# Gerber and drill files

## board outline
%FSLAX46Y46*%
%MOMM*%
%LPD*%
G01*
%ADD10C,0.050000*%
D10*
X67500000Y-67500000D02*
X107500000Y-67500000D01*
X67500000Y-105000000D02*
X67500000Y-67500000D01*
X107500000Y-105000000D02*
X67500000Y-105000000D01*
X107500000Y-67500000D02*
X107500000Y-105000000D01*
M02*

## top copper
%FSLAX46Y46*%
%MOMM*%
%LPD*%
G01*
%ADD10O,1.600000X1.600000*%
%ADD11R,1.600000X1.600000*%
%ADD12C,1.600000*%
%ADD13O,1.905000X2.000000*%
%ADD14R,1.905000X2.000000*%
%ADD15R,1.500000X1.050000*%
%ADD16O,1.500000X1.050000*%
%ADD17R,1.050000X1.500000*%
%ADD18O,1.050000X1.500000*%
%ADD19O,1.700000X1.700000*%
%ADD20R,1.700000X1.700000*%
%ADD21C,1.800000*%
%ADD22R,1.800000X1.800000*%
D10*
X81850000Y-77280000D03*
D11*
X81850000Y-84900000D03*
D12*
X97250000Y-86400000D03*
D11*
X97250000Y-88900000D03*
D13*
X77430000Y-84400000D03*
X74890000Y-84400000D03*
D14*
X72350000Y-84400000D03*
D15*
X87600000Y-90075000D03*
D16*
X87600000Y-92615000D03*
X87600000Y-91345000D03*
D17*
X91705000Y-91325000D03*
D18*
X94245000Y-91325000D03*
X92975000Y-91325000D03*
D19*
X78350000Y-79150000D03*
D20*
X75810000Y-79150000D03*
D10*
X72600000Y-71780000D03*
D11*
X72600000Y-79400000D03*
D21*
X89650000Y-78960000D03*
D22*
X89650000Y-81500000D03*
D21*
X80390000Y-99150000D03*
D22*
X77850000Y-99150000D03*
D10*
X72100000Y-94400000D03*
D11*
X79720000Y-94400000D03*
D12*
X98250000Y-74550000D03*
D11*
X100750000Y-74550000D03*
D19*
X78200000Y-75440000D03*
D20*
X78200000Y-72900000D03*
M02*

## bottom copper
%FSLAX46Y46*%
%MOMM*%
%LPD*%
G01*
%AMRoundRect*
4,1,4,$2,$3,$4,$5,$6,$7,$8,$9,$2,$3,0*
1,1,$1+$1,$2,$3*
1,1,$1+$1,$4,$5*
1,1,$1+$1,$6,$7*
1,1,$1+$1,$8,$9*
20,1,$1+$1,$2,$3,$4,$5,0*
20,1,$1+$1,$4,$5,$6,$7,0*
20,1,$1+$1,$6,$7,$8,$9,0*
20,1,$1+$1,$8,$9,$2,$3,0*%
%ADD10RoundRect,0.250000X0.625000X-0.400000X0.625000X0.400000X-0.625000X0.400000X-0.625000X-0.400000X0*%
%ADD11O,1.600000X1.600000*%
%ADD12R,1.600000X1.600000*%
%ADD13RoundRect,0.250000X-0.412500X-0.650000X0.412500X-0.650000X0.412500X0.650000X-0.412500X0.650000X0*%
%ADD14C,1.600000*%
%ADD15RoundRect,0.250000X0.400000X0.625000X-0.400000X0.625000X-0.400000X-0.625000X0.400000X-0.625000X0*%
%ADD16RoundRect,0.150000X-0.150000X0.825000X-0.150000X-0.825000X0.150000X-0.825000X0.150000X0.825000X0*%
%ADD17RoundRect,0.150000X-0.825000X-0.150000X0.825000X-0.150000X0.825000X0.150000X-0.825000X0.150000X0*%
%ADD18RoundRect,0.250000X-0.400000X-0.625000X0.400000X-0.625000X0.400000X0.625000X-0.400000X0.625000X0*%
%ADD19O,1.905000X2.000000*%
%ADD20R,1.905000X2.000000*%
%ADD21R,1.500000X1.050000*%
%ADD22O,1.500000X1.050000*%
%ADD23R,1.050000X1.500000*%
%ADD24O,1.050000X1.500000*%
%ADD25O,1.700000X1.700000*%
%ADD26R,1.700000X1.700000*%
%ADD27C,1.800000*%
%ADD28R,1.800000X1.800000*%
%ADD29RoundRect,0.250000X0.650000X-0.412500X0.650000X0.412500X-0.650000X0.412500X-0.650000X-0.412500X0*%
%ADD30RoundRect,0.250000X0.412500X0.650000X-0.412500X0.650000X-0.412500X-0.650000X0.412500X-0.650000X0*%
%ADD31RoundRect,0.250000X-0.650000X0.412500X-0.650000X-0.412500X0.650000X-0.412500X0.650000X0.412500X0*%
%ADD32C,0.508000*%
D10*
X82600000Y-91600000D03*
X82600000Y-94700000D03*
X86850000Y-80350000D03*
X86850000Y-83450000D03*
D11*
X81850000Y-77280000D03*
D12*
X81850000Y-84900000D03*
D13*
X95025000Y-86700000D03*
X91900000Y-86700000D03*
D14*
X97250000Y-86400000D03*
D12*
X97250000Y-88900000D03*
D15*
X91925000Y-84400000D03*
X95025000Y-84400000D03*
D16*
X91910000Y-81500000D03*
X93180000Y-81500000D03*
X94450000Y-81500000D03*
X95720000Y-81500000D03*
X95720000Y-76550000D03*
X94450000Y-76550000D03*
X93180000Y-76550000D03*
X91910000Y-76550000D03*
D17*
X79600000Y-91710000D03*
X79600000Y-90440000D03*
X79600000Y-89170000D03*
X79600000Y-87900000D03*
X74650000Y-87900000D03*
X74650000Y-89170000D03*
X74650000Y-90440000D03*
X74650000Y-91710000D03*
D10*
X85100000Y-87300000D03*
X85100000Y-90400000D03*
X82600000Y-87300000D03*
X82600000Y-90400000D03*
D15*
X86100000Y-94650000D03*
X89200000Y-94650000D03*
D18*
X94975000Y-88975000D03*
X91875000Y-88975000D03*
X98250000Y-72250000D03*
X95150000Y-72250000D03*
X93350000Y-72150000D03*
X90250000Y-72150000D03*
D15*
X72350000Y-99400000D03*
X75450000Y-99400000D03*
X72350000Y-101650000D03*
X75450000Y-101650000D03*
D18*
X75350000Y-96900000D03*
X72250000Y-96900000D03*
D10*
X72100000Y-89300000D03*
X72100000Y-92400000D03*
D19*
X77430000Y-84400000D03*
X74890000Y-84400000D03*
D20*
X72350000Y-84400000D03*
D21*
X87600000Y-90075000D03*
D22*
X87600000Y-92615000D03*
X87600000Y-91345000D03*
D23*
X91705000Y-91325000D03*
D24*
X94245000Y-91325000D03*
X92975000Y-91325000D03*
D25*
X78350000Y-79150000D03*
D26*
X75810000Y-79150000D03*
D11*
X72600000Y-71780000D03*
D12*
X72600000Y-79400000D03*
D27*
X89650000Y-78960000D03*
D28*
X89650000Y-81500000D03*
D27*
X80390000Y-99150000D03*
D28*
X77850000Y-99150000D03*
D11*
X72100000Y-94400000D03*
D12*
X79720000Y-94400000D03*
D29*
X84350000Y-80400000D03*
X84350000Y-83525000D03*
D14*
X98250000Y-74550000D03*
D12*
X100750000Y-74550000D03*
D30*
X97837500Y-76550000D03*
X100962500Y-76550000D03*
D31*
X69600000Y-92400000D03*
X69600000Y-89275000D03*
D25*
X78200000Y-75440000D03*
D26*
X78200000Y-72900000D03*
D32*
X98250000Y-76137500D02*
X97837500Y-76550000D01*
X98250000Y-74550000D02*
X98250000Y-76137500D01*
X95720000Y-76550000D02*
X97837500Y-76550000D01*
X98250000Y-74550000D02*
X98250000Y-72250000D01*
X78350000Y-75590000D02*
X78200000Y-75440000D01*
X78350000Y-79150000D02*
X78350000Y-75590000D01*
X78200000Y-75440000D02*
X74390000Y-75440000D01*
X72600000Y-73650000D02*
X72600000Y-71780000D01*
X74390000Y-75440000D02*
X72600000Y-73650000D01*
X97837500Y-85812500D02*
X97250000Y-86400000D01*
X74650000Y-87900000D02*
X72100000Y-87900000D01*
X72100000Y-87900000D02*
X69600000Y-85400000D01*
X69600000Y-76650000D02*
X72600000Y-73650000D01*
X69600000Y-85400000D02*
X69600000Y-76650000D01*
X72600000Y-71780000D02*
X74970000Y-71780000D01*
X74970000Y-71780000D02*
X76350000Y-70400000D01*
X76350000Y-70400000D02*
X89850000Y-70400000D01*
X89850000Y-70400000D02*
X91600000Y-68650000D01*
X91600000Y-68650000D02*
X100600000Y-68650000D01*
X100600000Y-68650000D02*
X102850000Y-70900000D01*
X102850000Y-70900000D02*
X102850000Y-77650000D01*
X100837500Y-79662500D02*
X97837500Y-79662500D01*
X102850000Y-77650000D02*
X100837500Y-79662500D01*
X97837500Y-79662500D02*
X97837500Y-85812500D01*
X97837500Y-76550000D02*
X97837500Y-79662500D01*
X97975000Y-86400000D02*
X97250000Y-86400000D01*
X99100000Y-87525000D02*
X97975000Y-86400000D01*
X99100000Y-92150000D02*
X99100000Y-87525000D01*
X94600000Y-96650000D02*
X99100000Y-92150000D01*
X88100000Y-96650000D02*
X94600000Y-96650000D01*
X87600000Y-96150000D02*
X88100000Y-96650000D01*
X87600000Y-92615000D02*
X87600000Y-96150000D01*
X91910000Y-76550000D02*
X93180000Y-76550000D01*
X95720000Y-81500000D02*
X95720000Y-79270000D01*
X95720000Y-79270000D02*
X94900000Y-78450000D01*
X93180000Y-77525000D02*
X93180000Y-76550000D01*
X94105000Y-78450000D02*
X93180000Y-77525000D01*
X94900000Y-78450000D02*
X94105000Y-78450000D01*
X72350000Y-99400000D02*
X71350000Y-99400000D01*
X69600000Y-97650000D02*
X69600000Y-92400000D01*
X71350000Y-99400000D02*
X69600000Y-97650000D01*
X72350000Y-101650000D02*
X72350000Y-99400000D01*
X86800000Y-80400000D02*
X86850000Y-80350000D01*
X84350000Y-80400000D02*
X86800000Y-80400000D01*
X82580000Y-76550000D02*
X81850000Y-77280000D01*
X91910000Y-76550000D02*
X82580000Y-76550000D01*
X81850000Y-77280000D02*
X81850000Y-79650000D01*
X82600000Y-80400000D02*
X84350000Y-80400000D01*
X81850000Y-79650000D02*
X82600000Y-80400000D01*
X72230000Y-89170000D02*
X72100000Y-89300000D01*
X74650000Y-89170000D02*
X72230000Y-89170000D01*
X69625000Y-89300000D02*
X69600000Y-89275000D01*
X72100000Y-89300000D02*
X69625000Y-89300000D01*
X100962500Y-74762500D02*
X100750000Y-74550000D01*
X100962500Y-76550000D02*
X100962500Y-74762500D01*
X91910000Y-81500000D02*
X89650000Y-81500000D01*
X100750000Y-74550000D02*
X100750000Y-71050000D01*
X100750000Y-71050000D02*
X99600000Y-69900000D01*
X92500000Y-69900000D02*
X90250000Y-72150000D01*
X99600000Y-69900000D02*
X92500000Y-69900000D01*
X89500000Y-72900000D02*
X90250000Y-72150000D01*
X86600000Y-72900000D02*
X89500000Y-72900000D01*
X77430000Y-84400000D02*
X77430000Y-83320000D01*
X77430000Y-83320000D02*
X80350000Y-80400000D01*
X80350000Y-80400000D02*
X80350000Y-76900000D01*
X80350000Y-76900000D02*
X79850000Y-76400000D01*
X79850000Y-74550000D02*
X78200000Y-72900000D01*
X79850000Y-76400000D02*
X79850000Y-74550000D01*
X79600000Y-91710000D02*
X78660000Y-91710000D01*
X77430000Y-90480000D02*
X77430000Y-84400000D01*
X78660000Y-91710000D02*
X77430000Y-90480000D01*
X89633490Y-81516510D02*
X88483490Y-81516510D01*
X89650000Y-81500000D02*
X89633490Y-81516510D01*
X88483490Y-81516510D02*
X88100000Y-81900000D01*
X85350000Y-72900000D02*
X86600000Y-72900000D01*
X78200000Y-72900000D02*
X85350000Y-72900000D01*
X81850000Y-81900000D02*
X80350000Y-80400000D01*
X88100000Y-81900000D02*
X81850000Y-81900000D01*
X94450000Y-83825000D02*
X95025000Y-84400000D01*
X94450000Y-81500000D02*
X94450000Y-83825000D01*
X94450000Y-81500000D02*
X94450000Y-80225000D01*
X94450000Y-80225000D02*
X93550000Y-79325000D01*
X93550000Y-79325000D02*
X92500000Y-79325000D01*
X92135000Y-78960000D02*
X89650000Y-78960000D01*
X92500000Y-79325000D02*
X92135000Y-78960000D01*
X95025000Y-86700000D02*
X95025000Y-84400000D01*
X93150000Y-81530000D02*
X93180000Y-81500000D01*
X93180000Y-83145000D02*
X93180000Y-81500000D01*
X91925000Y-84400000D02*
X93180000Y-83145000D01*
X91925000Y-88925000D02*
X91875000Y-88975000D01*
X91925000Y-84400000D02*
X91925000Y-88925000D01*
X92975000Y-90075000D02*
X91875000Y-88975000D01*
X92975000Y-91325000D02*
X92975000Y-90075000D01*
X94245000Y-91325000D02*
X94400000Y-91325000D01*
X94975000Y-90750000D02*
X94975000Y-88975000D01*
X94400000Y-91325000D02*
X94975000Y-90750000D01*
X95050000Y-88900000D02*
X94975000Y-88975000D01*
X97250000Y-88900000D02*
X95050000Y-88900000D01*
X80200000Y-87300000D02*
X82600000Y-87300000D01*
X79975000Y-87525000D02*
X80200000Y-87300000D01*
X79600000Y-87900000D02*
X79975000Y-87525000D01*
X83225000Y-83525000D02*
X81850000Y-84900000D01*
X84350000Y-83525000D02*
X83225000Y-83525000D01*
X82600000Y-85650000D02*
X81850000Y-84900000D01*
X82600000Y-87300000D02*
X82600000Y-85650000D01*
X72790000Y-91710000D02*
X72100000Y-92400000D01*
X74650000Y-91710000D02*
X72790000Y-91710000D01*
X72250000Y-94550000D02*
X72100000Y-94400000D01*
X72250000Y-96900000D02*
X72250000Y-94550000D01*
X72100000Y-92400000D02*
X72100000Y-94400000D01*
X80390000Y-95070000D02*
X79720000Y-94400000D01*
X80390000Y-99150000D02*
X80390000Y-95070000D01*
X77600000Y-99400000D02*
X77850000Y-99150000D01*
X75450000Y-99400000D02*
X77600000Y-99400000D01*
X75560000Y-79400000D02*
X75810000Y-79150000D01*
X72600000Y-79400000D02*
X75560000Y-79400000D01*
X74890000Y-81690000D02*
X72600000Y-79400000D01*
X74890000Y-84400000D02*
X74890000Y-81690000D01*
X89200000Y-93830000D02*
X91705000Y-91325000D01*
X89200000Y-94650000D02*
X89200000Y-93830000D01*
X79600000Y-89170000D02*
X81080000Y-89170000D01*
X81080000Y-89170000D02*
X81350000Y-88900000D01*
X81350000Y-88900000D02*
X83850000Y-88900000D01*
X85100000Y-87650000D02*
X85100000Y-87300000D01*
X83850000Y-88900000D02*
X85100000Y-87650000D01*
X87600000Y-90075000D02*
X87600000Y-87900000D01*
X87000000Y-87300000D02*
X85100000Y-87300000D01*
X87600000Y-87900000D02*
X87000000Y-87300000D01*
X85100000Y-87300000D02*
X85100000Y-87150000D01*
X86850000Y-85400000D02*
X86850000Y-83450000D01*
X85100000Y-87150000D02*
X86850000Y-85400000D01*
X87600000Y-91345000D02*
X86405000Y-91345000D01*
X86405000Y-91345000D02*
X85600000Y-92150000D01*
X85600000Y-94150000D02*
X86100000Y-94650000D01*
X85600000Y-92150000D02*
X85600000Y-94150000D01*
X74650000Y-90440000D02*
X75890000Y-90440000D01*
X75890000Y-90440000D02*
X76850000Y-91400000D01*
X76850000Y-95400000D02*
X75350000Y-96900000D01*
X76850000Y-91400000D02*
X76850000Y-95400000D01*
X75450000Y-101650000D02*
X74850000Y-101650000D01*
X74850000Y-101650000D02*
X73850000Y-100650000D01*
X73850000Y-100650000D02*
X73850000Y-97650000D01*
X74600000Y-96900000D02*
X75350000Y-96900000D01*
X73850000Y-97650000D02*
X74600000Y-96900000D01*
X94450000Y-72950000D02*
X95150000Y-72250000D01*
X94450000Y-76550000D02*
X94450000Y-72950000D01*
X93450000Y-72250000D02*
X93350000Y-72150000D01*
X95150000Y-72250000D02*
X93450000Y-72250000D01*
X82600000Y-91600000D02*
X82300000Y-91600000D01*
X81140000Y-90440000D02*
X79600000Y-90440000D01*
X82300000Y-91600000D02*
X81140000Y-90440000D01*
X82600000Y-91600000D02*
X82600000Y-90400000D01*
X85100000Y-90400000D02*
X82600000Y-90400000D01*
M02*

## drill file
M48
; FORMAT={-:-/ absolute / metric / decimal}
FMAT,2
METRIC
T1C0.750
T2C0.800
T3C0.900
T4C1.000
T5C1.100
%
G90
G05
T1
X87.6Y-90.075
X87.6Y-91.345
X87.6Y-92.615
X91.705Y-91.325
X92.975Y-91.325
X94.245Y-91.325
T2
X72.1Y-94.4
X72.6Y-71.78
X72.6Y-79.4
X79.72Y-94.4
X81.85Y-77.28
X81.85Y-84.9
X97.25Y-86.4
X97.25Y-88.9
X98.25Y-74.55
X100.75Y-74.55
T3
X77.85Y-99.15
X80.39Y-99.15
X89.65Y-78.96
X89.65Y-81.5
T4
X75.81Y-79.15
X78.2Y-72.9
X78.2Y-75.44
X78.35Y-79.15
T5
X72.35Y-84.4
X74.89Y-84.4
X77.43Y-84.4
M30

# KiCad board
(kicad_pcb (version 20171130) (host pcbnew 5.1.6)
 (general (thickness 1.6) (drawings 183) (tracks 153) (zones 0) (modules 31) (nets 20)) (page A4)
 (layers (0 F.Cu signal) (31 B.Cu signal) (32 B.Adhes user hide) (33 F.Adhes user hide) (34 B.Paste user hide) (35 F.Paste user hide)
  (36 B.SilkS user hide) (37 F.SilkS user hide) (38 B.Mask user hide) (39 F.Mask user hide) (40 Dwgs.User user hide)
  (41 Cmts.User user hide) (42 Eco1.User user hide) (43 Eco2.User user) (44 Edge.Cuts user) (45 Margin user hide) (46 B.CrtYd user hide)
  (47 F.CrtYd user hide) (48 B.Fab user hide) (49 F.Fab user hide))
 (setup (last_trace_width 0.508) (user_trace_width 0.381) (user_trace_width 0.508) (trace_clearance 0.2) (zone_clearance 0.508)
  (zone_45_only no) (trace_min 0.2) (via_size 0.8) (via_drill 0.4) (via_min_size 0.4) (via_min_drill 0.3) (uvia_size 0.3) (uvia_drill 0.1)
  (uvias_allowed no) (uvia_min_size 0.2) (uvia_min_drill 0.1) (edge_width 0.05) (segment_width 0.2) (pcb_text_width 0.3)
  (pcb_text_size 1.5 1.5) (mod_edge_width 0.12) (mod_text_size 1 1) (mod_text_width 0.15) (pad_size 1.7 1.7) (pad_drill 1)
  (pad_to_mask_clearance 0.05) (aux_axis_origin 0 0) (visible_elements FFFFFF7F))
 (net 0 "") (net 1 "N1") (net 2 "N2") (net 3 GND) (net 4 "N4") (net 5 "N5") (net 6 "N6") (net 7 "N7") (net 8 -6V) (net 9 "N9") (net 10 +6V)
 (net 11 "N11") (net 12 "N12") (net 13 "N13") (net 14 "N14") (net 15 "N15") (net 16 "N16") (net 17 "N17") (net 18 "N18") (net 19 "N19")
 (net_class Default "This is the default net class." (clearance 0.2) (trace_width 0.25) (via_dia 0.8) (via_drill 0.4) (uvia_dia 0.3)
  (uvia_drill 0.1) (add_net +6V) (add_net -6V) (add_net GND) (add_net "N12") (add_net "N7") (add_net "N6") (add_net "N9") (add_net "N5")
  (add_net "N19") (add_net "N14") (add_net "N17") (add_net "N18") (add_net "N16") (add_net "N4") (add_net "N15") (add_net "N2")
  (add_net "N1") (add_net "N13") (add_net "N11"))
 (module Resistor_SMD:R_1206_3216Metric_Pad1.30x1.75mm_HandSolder (layer B.Cu) (at 82.6 93.15 90)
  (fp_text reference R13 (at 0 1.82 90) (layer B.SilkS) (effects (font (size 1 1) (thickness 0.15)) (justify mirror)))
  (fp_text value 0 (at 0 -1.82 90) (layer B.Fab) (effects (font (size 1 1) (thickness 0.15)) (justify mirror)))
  (pad 2 smd roundrect (at 1.55 0 90) (size 1.3 1.75) (layers B.Cu B.Paste B.Mask) (roundrect_rratio 0.192308) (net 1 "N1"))
  (pad 1 smd roundrect (at -1.55 0 90) (size 1.3 1.75) (layers B.Cu B.Paste B.Mask) (roundrect_rratio 0.192308) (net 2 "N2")))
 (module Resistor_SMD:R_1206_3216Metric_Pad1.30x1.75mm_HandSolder (layer B.Cu) (at 86.85 81.9 90)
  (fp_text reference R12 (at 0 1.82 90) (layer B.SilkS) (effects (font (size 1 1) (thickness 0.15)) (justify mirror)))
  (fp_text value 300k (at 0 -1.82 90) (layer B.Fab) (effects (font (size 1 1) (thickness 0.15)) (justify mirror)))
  (pad 2 smd roundrect (at 1.55 0 90) (size 1.3 1.75) (layers B.Cu B.Paste B.Mask) (roundrect_rratio 0.192308) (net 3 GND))
  (pad 1 smd roundrect (at -1.55 0 90) (size 1.3 1.75) (layers B.Cu B.Paste B.Mask) (roundrect_rratio 0.192308) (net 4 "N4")))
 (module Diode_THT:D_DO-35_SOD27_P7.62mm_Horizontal (layer F.Cu) (at 81.85 84.9 90)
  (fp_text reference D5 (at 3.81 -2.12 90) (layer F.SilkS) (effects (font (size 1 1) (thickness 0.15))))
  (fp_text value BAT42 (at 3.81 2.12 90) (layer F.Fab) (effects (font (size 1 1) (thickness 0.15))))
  (pad 2 thru_hole oval (at 7.62 0 90) (size 1.6 1.6) (drill 0.8) (layers *.Cu *.Mask) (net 3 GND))
  (pad 1 thru_hole rect (at 0 0 90) (size 1.6 1.6) (drill 0.8) (layers *.Cu *.Mask) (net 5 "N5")))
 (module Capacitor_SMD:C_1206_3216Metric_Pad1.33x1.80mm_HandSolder (layer B.Cu) (at 93.4625 86.7)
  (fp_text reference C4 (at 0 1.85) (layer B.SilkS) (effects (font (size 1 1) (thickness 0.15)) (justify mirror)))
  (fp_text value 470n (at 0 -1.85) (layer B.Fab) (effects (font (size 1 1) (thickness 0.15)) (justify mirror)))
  (pad 2 smd roundrect (at 1.5625 0) (size 1.325 1.8) (layers B.Cu B.Paste B.Mask) (roundrect_rratio 0.188679) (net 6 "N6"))
  (pad 1 smd roundrect (at -1.5625 0) (size 1.325 1.8) (layers B.Cu B.Paste B.Mask) (roundrect_rratio 0.188679) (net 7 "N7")))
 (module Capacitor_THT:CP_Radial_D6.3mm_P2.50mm (layer F.Cu) (at 97.25 88.9 90)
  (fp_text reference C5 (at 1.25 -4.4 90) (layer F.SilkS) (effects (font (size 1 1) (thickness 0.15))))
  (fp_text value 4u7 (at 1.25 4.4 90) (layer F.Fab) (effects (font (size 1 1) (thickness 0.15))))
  (pad 2 thru_hole circle (at 2.5 0 90) (size 1.6 1.6) (drill 0.8) (layers *.Cu *.Mask) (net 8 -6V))
  (pad 1 thru_hole rect (at 0 0 90) (size 1.6 1.6) (drill 0.8) (layers *.Cu *.Mask) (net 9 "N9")))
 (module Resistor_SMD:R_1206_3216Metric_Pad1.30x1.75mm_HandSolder (layer B.Cu) (at 93.475 84.4 180)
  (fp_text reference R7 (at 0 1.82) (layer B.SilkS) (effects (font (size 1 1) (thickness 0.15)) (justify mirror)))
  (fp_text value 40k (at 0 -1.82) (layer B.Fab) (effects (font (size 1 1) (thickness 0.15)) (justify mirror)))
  (pad 2 smd roundrect (at 1.55 0 180) (size 1.3 1.75) (layers B.Cu B.Paste B.Mask) (roundrect_rratio 0.192308) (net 7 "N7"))
  (pad 1 smd roundrect (at -1.55 0 180) (size 1.3 1.75) (layers B.Cu B.Paste B.Mask) (roundrect_rratio 0.192308) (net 6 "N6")))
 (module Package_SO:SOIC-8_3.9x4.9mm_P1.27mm (layer B.Cu) (at 93.815 79.025 270)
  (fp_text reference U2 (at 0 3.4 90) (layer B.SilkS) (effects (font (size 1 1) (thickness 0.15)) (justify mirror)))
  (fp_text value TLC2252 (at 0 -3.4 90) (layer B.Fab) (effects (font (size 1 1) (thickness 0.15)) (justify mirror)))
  (pad 8 smd roundrect (at 2.475 1.905 270) (size 1.95 0.6) (layers B.Cu B.Paste B.Mask) (roundrect_rratio 0.25) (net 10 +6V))
  (pad 7 smd roundrect (at 2.475 0.635 270) (size 1.95 0.6) (layers B.Cu B.Paste B.Mask) (roundrect_rratio 0.25) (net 7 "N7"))
  (pad 6 smd roundrect (at 2.475 -0.635 270) (size 1.95 0.6) (layers B.Cu B.Paste B.Mask) (roundrect_rratio 0.25) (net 6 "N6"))
  (pad 5 smd roundrect (at 2.475 -1.905 270) (size 1.95 0.6) (layers B.Cu B.Paste B.Mask) (roundrect_rratio 0.25) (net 3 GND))
  (pad 4 smd roundrect (at -2.475 -1.905 270) (size 1.95 0.6) (layers B.Cu B.Paste B.Mask) (roundrect_rratio 0.25) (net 8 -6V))
  (pad 3 smd roundrect (at -2.475 -0.635 270) (size 1.95 0.6) (layers B.Cu B.Paste B.Mask) (roundrect_rratio 0.25) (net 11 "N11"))
  (pad 2 smd roundrect (at -2.475 0.635 270) (size 1.95 0.6) (layers B.Cu B.Paste B.Mask) (roundrect_rratio 0.25) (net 3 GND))
  (pad 1 smd roundrect (at -2.475 1.905 270) (size 1.95 0.6) (layers B.Cu B.Paste B.Mask) (roundrect_rratio 0.25) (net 3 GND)))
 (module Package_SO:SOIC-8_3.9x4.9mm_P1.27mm (layer B.Cu) (at 77.125 89.805)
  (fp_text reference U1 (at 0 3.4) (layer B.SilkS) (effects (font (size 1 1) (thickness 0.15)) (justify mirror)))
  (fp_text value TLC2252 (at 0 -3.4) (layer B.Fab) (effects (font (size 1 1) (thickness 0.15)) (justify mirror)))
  (pad 8 smd roundrect (at 2.475 1.905) (size 1.95 0.6) (layers B.Cu B.Paste B.Mask) (roundrect_rratio 0.25) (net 10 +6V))
  (pad 7 smd roundrect (at 2.475 0.635) (size 1.95 0.6) (layers B.Cu B.Paste B.Mask) (roundrect_rratio 0.25) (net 1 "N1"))
  (pad 6 smd roundrect (at 2.475 -0.635) (size 1.95 0.6) (layers B.Cu B.Paste B.Mask) (roundrect_rratio 0.25) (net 4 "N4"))
  (pad 5 smd roundrect (at 2.475 -1.905) (size 1.95 0.6) (layers B.Cu B.Paste B.Mask) (roundrect_rratio 0.25) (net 5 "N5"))
  (pad 4 smd roundrect (at -2.475 -1.905) (size 1.95 0.6) (layers B.Cu B.Paste B.Mask) (roundrect_rratio 0.25) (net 8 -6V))
  (pad 3 smd roundrect (at -2.475 -0.635) (size 1.95 0.6) (layers B.Cu B.Paste B.Mask) (roundrect_rratio 0.25) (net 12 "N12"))
  (pad 2 smd roundrect (at -2.475 0.635) (size 1.95 0.6) (layers B.Cu B.Paste B.Mask) (roundrect_rratio 0.25) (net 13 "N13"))
  (pad 1 smd roundrect (at -2.475 1.905) (size 1.95 0.6) (layers B.Cu B.Paste B.Mask) (roundrect_rratio 0.25) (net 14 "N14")))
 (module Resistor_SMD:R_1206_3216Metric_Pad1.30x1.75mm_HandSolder (layer B.Cu) (at 85.1 88.85 90)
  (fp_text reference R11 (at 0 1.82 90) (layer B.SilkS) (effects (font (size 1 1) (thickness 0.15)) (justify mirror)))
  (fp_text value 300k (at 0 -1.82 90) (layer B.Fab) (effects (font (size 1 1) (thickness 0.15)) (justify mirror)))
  (pad 2 smd roundrect (at 1.55 0 90) (size 1.3 1.75) (layers B.Cu B.Paste B.Mask) (roundrect_rratio 0.192308) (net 4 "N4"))
  (pad 1 smd roundrect (at -1.55 0 90) (size 1.3 1.75) (layers B.Cu B.Paste B.Mask) (roundrect_rratio 0.192308) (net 1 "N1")))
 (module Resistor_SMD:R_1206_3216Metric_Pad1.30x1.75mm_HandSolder (layer B.Cu) (at 82.6 88.85 90)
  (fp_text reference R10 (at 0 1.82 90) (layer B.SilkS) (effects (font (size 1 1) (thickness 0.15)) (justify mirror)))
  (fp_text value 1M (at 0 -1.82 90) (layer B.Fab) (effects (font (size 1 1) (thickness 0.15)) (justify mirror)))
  (pad 2 smd roundrect (at 1.55 0 90) (size 1.3 1.75) (layers B.Cu B.Paste B.Mask) (roundrect_rratio 0.192308) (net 5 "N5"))
  (pad 1 smd roundrect (at -1.55 0 90) (size 1.3 1.75) (layers B.Cu B.Paste B.Mask) (roundrect_rratio 0.192308) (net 1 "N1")))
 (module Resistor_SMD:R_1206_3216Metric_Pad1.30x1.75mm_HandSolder (layer B.Cu) (at 87.65 94.65 180)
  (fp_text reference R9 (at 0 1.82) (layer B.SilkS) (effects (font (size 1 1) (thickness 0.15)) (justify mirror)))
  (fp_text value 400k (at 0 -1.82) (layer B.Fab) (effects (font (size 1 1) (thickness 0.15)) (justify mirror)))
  (pad 2 smd roundrect (at 1.55 0 180) (size 1.3 1.75) (layers B.Cu B.Paste B.Mask) (roundrect_rratio 0.192308) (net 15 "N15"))
  (pad 1 smd roundrect (at -1.55 0 180) (size 1.3 1.75) (layers B.Cu B.Paste B.Mask) (roundrect_rratio 0.192308) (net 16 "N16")))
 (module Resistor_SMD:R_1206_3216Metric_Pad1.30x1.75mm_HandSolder (layer B.Cu) (at 93.425 88.975)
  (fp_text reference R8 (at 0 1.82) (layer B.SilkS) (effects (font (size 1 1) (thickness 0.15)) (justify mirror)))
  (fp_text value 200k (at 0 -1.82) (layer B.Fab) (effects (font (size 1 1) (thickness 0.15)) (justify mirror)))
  (pad 2 smd roundrect (at 1.55 0) (size 1.3 1.75) (layers B.Cu B.Paste B.Mask) (roundrect_rratio 0.192308) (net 9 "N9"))
  (pad 1 smd roundrect (at -1.55 0) (size 1.3 1.75) (layers B.Cu B.Paste B.Mask) (roundrect_rratio 0.192308) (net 7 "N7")))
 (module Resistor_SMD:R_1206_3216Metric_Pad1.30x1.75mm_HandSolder (layer B.Cu) (at 96.7 72.25)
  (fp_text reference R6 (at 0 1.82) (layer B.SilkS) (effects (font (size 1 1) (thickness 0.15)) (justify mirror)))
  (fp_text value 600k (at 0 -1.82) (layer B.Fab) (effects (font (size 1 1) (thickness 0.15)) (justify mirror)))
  (pad 2 smd roundrect (at 1.55 0) (size 1.3 1.75) (layers B.Cu B.Paste B.Mask) (roundrect_rratio 0.192308) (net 8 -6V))
  (pad 1 smd roundrect (at -1.55 0) (size 1.3 1.75) (layers B.Cu B.Paste B.Mask) (roundrect_rratio 0.192308) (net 11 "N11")))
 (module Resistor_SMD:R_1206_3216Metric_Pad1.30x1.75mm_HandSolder (layer B.Cu) (at 91.8 72.15)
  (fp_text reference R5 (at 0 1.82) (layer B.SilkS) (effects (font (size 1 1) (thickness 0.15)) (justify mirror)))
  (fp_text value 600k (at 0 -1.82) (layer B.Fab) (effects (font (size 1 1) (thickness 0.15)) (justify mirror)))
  (pad 2 smd roundrect (at 1.55 0) (size 1.3 1.75) (layers B.Cu B.Paste B.Mask) (roundrect_rratio 0.192308) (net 11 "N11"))
  (pad 1 smd roundrect (at -1.55 0) (size 1.3 1.75) (layers B.Cu B.Paste B.Mask) (roundrect_rratio 0.192308) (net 10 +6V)))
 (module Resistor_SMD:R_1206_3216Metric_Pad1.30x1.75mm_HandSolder (layer B.Cu) (at 73.9 99.4 180)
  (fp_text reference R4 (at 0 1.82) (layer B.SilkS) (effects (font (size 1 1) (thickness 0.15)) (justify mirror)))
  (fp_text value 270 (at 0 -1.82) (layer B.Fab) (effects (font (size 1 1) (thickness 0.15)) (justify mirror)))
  (pad 2 smd roundrect (at 1.55 0 180) (size 1.3 1.75) (layers B.Cu B.Paste B.Mask) (roundrect_rratio 0.192308) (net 3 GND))
  (pad 1 smd roundrect (at -1.55 0 180) (size 1.3 1.75) (layers B.Cu B.Paste B.Mask) (roundrect_rratio 0.192308) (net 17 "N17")))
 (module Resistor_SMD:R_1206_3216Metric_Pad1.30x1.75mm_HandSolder (layer B.Cu) (at 73.9 101.65 180)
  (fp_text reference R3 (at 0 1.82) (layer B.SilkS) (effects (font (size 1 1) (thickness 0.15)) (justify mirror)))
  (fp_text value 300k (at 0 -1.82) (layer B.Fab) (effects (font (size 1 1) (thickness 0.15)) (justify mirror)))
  (pad 2 smd roundrect (at 1.55 0 180) (size 1.3 1.75) (layers B.Cu B.Paste B.Mask) (roundrect_rratio 0.192308) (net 3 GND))
  (pad 1 smd roundrect (at -1.55 0 180) (size 1.3 1.75) (layers B.Cu B.Paste B.Mask) (roundrect_rratio 0.192308) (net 13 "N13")))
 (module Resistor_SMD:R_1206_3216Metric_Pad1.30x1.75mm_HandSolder (layer B.Cu) (at 73.8 96.9)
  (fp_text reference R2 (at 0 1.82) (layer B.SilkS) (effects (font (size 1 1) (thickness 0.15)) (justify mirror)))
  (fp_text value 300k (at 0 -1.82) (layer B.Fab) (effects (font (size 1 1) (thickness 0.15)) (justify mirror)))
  (pad 2 smd roundrect (at 1.55 0) (size 1.3 1.75) (layers B.Cu B.Paste B.Mask) (roundrect_rratio 0.192308) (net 13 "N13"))
  (pad 1 smd roundrect (at -1.55 0) (size 1.3 1.75) (layers B.Cu B.Paste B.Mask) (roundrect_rratio 0.192308) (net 14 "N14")))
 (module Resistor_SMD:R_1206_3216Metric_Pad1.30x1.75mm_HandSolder (layer B.Cu) (at 72.1 90.85 90)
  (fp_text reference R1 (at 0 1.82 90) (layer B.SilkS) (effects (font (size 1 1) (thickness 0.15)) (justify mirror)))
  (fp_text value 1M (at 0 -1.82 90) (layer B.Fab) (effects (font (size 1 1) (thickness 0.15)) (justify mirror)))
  (pad 2 smd roundrect (at 1.55 0 90) (size 1.3 1.75) (layers B.Cu B.Paste B.Mask) (roundrect_rratio 0.192308) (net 12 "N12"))
  (pad 1 smd roundrect (at -1.55 0 90) (size 1.3 1.75) (layers B.Cu B.Paste B.Mask) (roundrect_rratio 0.192308) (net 14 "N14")))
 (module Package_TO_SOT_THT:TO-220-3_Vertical (layer F.Cu) (at 72.35 84.4)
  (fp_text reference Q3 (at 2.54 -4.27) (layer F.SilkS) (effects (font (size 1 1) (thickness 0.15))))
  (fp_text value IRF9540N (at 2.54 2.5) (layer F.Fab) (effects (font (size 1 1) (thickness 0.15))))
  (pad 3 thru_hole oval (at 5.08 0) (size 1.905 2) (drill 1.1) (layers *.Cu *.Mask) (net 10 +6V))
  (pad 2 thru_hole oval (at 2.54 0) (size 1.905 2) (drill 1.1) (layers *.Cu *.Mask) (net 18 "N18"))
  (pad 1 thru_hole rect (at 0 0) (size 1.905 2) (drill 1.1) (layers *.Cu *.Mask) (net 2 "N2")))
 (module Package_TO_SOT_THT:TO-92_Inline (layer F.Cu) (at 87.6 90.075 270)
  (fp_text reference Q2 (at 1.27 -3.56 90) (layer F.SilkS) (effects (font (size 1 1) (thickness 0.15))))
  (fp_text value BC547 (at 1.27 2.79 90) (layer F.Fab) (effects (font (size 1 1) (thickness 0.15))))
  (pad 1 thru_hole rect (at 0 0 270) (size 1.05 1.5) (drill 0.75) (layers *.Cu *.Mask) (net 4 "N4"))
  (pad 3 thru_hole oval (at 2.54 0 270) (size 1.05 1.5) (drill 0.75) (layers *.Cu *.Mask) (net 8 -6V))
  (pad 2 thru_hole oval (at 1.27 0 270) (size 1.05 1.5) (drill 0.75) (layers *.Cu *.Mask) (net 15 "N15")))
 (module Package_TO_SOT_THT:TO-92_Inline (layer F.Cu) (at 91.705 91.325)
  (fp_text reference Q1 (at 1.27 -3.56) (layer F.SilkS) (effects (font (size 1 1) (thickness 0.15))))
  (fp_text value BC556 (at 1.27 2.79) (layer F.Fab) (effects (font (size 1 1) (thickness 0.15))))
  (pad 1 thru_hole rect (at 0 0) (size 1.05 1.5) (drill 0.75) (layers *.Cu *.Mask) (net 16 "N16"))
  (pad 3 thru_hole oval (at 2.54 0) (size 1.05 1.5) (drill 0.75) (layers *.Cu *.Mask) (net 9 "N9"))
  (pad 2 thru_hole oval (at 1.27 0) (size 1.05 1.5) (drill 0.75) (layers *.Cu *.Mask) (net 7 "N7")))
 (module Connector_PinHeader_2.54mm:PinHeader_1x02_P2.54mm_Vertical (layer F.Cu) (at 75.81 79.15 90)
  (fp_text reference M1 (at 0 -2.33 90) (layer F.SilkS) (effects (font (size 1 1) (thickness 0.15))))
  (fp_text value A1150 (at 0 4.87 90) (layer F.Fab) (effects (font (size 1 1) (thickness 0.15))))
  (pad 2 thru_hole oval (at 0 2.54 90) (size 1.7 1.7) (drill 1) (layers *.Cu *.Mask) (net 8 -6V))
  (pad 1 thru_hole rect (at 0 0 90) (size 1.7 1.7) (drill 1) (layers *.Cu *.Mask) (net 18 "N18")))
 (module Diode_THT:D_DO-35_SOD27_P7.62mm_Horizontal (layer F.Cu) (at 72.6 79.4 90)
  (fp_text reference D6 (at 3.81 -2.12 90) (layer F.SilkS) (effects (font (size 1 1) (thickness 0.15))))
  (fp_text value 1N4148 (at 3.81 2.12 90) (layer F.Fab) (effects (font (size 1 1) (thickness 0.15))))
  (pad 2 thru_hole oval (at 7.62 0 90) (size 1.6 1.6) (drill 0.8) (layers *.Cu *.Mask) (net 8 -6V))
  (pad 1 thru_hole rect (at 0 0 90) (size 1.6 1.6) (drill 0.8) (layers *.Cu *.Mask) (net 18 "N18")))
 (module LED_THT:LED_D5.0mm (layer F.Cu) (at 89.65 81.5 90)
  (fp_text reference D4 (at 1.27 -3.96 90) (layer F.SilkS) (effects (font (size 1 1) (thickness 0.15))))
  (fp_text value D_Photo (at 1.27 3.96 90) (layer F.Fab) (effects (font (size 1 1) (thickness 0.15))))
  (pad 2 thru_hole circle (at 2.54 0 90) (size 1.8 1.8) (drill 0.9) (layers *.Cu *.Mask) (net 6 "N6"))
  (pad 1 thru_hole rect (at 0 0 90) (size 1.8 1.8) (drill 0.9) (layers *.Cu *.Mask) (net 10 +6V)))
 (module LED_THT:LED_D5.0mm (layer F.Cu) (at 77.85 99.15)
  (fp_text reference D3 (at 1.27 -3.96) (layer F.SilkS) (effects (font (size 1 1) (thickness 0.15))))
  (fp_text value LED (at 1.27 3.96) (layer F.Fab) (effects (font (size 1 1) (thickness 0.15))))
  (pad 2 thru_hole circle (at 2.54 0) (size 1.8 1.8) (drill 0.9) (layers *.Cu *.Mask) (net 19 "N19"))
  (pad 1 thru_hole rect (at 0 0) (size 1.8 1.8) (drill 0.9) (layers *.Cu *.Mask) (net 17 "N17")))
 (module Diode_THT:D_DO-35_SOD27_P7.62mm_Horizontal (layer F.Cu) (at 79.72 94.4 180)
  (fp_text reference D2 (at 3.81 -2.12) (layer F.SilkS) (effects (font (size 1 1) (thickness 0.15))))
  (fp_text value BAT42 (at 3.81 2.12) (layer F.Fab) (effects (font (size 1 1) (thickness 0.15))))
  (pad 2 thru_hole oval (at 7.62 0 180) (size 1.6 1.6) (drill 0.8) (layers *.Cu *.Mask) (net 14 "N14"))
  (pad 1 thru_hole rect (at 0 0 180) (size 1.6 1.6) (drill 0.8) (layers *.Cu *.Mask) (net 19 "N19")))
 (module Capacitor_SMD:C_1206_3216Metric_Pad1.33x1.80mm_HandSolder (layer B.Cu) (at 84.35 81.9625 90)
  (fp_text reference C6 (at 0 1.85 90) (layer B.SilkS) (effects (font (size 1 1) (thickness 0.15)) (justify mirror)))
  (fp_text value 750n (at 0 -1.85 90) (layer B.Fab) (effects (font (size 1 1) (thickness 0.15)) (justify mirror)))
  (pad 2 smd roundrect (at 1.5625 0 90) (size 1.325 1.8) (layers B.Cu B.Paste B.Mask) (roundrect_rratio 0.188679) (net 3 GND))
  (pad 1 smd roundrect (at -1.5625 0 90) (size 1.325 1.8) (layers B.Cu B.Paste B.Mask) (roundrect_rratio 0.188679) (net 5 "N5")))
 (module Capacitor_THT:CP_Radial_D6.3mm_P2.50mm (layer F.Cu) (at 100.75 74.55 180)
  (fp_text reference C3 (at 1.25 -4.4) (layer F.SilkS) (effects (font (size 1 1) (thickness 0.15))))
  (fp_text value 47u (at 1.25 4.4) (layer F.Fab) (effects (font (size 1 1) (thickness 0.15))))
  (pad 2 thru_hole circle (at 2.5 0 180) (size 1.6 1.6) (drill 0.8) (layers *.Cu *.Mask) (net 8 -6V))
  (pad 1 thru_hole rect (at 0 0 180) (size 1.6 1.6) (drill 0.8) (layers *.Cu *.Mask) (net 10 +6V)))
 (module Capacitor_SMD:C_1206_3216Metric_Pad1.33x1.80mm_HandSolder (layer B.Cu) (at 99.4 76.55 180)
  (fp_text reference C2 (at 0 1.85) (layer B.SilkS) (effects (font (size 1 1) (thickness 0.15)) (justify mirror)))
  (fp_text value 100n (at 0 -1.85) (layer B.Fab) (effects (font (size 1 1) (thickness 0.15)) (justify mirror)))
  (pad 2 smd roundrect (at 1.5625 0 180) (size 1.325 1.8) (layers B.Cu B.Paste B.Mask) (roundrect_rratio 0.188679) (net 8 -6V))
  (pad 1 smd roundrect (at -1.5625 0 180) (size 1.325 1.8) (layers B.Cu B.Paste B.Mask) (roundrect_rratio 0.188679) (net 10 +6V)))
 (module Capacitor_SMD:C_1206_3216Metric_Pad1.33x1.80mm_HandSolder (layer B.Cu) (at 69.6 90.8375 270)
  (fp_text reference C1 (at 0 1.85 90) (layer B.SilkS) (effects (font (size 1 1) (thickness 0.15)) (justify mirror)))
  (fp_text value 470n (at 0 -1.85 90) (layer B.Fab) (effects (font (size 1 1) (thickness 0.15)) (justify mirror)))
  (pad 2 smd roundrect (at 1.5625 0 270) (size 1.325 1.8) (layers B.Cu B.Paste B.Mask) (roundrect_rratio 0.188679) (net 3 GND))
  (pad 1 smd roundrect (at -1.5625 0 270) (size 1.325 1.8) (layers B.Cu B.Paste B.Mask) (roundrect_rratio 0.188679) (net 12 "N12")))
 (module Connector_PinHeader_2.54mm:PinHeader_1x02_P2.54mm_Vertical (layer F.Cu) (at 78.2 72.9)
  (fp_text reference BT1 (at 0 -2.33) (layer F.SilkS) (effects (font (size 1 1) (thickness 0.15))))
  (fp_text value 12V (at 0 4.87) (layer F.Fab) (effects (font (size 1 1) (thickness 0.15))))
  (pad 2 thru_hole oval (at 0 2.54) (size 1.7 1.7) (drill 1) (layers *.Cu *.Mask) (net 8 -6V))
  (pad 1 thru_hole rect (at 0 0) (size 1.7 1.7) (drill 1) (layers *.Cu *.Mask) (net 10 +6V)))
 (gr_line (start 67.5 67.5) (end 107.5 67.5) (layer Edge.Cuts) (width 0.05))
 (gr_line (start 67.5 105) (end 67.5 67.5) (layer Edge.Cuts) (width 0.05))
 (gr_line (start 107.5 105) (end 67.5 105) (layer Edge.Cuts) (width 0.05))
 (gr_line (start 107.5 67.5) (end 107.5 105) (layer Edge.Cuts) (width 0.05))
 (segment (start 98.25 76.1375) (end 97.8375 76.55) (width 0.508) (layer B.Cu) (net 8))
 (segment (start 98.25 74.55) (end 98.25 76.1375) (width 0.508) (layer B.Cu) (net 8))
 (segment (start 95.72 76.55) (end 97.8375 76.55) (width 0.508) (layer B.Cu) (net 8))
 (segment (start 98.25 74.55) (end 98.25 72.25) (width 0.508) (layer B.Cu) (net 8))
 (segment (start 78.35 75.59) (end 78.2 75.44) (width 0.508) (layer B.Cu) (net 8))
 (segment (start 78.35 79.15) (end 78.35 75.59) (width 0.508) (layer B.Cu) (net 8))
 (segment (start 78.2 75.44) (end 74.39 75.44) (width 0.508) (layer B.Cu) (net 8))
 (segment (start 72.6 73.65) (end 72.6 71.78) (width 0.508) (layer B.Cu) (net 8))
 (segment (start 74.39 75.44) (end 72.6 73.65) (width 0.508) (layer B.Cu) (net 8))
 (segment (start 97.8375 85.8125) (end 97.25 86.4) (width 0.508) (layer B.Cu) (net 8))
 (segment (start 74.65 87.9) (end 72.1 87.9) (width 0.508) (layer B.Cu) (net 8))
 (segment (start 72.1 87.9) (end 69.6 85.4) (width 0.508) (layer B.Cu) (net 8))
 (segment (start 69.6 76.65) (end 72.6 73.65) (width 0.508) (layer B.Cu) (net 8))
 (segment (start 69.6 85.4) (end 69.6 76.65) (width 0.508) (layer B.Cu) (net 8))
 (segment (start 72.6 71.78) (end 74.97 71.78) (width 0.508) (layer B.Cu) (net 8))
 (segment (start 74.97 71.78) (end 76.35 70.4) (width 0.508) (layer B.Cu) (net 8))
 (segment (start 76.35 70.4) (end 89.85 70.4) (width 0.508) (layer B.Cu) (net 8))
 (segment (start 89.85 70.4) (end 91.6 68.65) (width 0.508) (layer B.Cu) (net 8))
 (segment (start 91.6 68.65) (end 100.6 68.65) (width 0.508) (layer B.Cu) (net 8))
 (segment (start 100.6 68.65) (end 102.85 70.9) (width 0.508) (layer B.Cu) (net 8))
 (segment (start 102.85 70.9) (end 102.85 77.65) (width 0.508) (layer B.Cu) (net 8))
 (segment (start 100.8375 79.6625) (end 97.8375 79.6625) (width 0.508) (layer B.Cu) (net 8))
 (segment (start 102.85 77.65) (end 100.8375 79.6625) (width 0.508) (layer B.Cu) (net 8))
 (segment (start 97.8375 79.6625) (end 97.8375 85.8125) (width 0.508) (layer B.Cu) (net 8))
 (segment (start 97.8375 76.55) (end 97.8375 79.6625) (width 0.508) (layer B.Cu) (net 8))
 (segment (start 97.975 86.4) (end 97.25 86.4) (width 0.508) (layer B.Cu) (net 8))
 (segment (start 99.1 87.525) (end 97.975 86.4) (width 0.508) (layer B.Cu) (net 8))
 (segment (start 99.1 92.15) (end 99.1 87.525) (width 0.508) (layer B.Cu) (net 8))
 (segment (start 94.6 96.65) (end 99.1 92.15) (width 0.508) (layer B.Cu) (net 8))
 (segment (start 88.1 96.65) (end 94.6 96.65) (width 0.508) (layer B.Cu) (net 8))
 (segment (start 87.6 96.15) (end 88.1 96.65) (width 0.508) (layer B.Cu) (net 8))
 (segment (start 87.6 92.615) (end 87.6 96.15) (width 0.508) (layer B.Cu) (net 8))
 (segment (start 91.91 76.55) (end 93.18 76.55) (width 0.508) (layer B.Cu) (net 3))
 (segment (start 95.72 81.5) (end 95.72 79.27) (width 0.508) (layer B.Cu) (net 3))
 (segment (start 95.72 79.27) (end 94.9 78.45) (width 0.508) (layer B.Cu) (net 3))
 (segment (start 93.18 77.525) (end 93.18 76.55) (width 0.508) (layer B.Cu) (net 3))
 (segment (start 94.105 78.45) (end 93.18 77.525) (width 0.508) (layer B.Cu) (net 3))
 (segment (start 94.9 78.45) (end 94.105 78.45) (width 0.508) (layer B.Cu) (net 3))
 (segment (start 72.35 99.4) (end 71.35 99.4) (width 0.508) (layer B.Cu) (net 3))
 (segment (start 69.6 97.65) (end 69.6 92.4) (width 0.508) (layer B.Cu) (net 3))
 (segment (start 71.35 99.4) (end 69.6 97.65) (width 0.508) (layer B.Cu) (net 3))
 (segment (start 72.35 101.65) (end 72.35 99.4) (width 0.508) (layer B.Cu) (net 3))
 (segment (start 86.8 80.4) (end 86.85 80.35) (width 0.508) (layer B.Cu) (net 3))
 (segment (start 84.35 80.4) (end 86.8 80.4) (width 0.508) (layer B.Cu) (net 3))
 (segment (start 82.58 76.55) (end 81.85 77.28) (width 0.508) (layer B.Cu) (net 3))
 (segment (start 91.91 76.55) (end 82.58 76.55) (width 0.508) (layer B.Cu) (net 3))
 (segment (start 81.85 77.28) (end 81.85 79.65) (width 0.508) (layer B.Cu) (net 3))
 (segment (start 82.6 80.4) (end 84.35 80.4) (width 0.508) (layer B.Cu) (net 3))
 (segment (start 81.85 79.65) (end 82.6 80.4) (width 0.508) (layer B.Cu) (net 3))
 (segment (start 72.23 89.17) (end 72.1 89.3) (width 0.508) (layer B.Cu) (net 12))
 (segment (start 74.65 89.17) (end 72.23 89.17) (width 0.508) (layer B.Cu) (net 12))
 (segment (start 69.625 89.3) (end 69.6 89.275) (width 0.508) (layer B.Cu) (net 12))
 (segment (start 72.1 89.3) (end 69.625 89.3) (width 0.508) (layer B.Cu) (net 12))
 (segment (start 100.9625 74.7625) (end 100.75 74.55) (width 0.508) (layer B.Cu) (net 10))
 (segment (start 100.9625 76.55) (end 100.9625 74.7625) (width 0.508) (layer B.Cu) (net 10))
 (segment (start 91.91 81.5) (end 89.65 81.5) (width 0.508) (layer B.Cu) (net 10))
 (segment (start 100.75 74.55) (end 100.75 71.05) (width 0.508) (layer B.Cu) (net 10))
 (segment (start 100.75 71.05) (end 99.6 69.9) (width 0.508) (layer B.Cu) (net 10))
 (segment (start 92.5 69.9) (end 90.25 72.15) (width 0.508) (layer B.Cu) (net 10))
 (segment (start 99.6 69.9) (end 92.5 69.9) (width 0.508) (layer B.Cu) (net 10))
 (segment (start 89.5 72.9) (end 90.25 72.15) (width 0.508) (layer B.Cu) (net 10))
 (segment (start 86.6 72.9) (end 89.5 72.9) (width 0.508) (layer B.Cu) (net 10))
 (segment (start 77.43 84.4) (end 77.43 83.32) (width 0.508) (layer B.Cu) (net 10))
 (segment (start 77.43 83.32) (end 80.35 80.4) (width 0.508) (layer B.Cu) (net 10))
 (segment (start 80.35 80.4) (end 80.35 76.9) (width 0.508) (layer B.Cu) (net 10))
 (segment (start 80.35 76.9) (end 79.85 76.4) (width 0.508) (layer B.Cu) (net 10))
 (segment (start 79.85 74.55) (end 78.2 72.9) (width 0.508) (layer B.Cu) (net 10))
 (segment (start 79.85 76.4) (end 79.85 74.55) (width 0.508) (layer B.Cu) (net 10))
 (segment (start 79.6 91.71) (end 78.66 91.71) (width 0.508) (layer B.Cu) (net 10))
 (segment (start 77.43 90.48) (end 77.43 84.4) (width 0.508) (layer B.Cu) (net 10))
 (segment (start 78.66 91.71) (end 77.43 90.48) (width 0.508) (layer B.Cu) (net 10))
 (segment (start 89.63349 81.51651) (end 88.48349 81.51651) (width 0.508) (layer B.Cu) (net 10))
 (segment (start 89.65 81.5) (end 89.63349 81.51651) (width 0.508) (layer B.Cu) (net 10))
 (segment (start 88.48349 81.51651) (end 88.1 81.9) (width 0.508) (layer B.Cu) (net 10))
 (segment (start 85.35 72.9) (end 86.6 72.9) (width 0.508) (layer B.Cu) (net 10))
 (segment (start 78.2 72.9) (end 85.35 72.9) (width 0.508) (layer B.Cu) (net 10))
 (segment (start 81.85 81.9) (end 80.35 80.4) (width 0.508) (layer B.Cu) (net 10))
 (segment (start 88.1 81.9) (end 81.85 81.9) (width 0.508) (layer B.Cu) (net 10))
 (segment (start 94.45 83.825) (end 95.025 84.4) (width 0.508) (layer B.Cu) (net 6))
 (segment (start 94.45 81.5) (end 94.45 83.825) (width 0.508) (layer B.Cu) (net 6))
 (segment (start 94.45 81.5) (end 94.45 80.225) (width 0.508) (layer B.Cu) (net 6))
 (segment (start 94.45 80.225) (end 93.55 79.325) (width 0.508) (layer B.Cu) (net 6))
 (segment (start 93.55 79.325) (end 92.5 79.325) (width 0.508) (layer B.Cu) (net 6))
 (segment (start 92.135 78.96) (end 89.65 78.96) (width 0.508) (layer B.Cu) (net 6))
 (segment (start 92.5 79.325) (end 92.135 78.96) (width 0.508) (layer B.Cu) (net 6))
 (segment (start 95.025 86.7) (end 95.025 84.4) (width 0.508) (layer B.Cu) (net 6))
 (segment (start 93.15 81.53) (end 93.18 81.5) (width 0.508) (layer B.Cu) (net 7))
 (segment (start 93.18 83.145) (end 93.18 81.5) (width 0.508) (layer B.Cu) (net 7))
 (segment (start 91.925 84.4) (end 93.18 83.145) (width 0.508) (layer B.Cu) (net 7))
 (segment (start 91.925 88.925) (end 91.875 88.975) (width 0.508) (layer B.Cu) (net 7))
 (segment (start 91.925 84.4) (end 91.925 88.925) (width 0.508) (layer B.Cu) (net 7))
 (segment (start 92.975 90.075) (end 91.875 88.975) (width 0.508) (layer B.Cu) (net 7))
 (segment (start 92.975 91.325) (end 92.975 90.075) (width 0.508) (layer B.Cu) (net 7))
 (segment (start 94.245 91.325) (end 94.4 91.325) (width 0.508) (layer B.Cu) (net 9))
 (segment (start 94.975 90.75) (end 94.975 88.975) (width 0.508) (layer B.Cu) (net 9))
 (segment (start 94.4 91.325) (end 94.975 90.75) (width 0.508) (layer B.Cu) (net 9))
 (segment (start 95.05 88.9) (end 94.975 88.975) (width 0.508) (layer B.Cu) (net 9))
 (segment (start 97.25 88.9) (end 95.05 88.9) (width 0.508) (layer B.Cu) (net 9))
 (segment (start 80.2 87.3) (end 82.6 87.3) (width 0.508) (layer B.Cu) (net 5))
 (segment (start 79.975 87.525) (end 80.2 87.3) (width 0.508) (layer B.Cu) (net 5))
 (segment (start 79.6 87.9) (end 79.975 87.525) (width 0.508) (layer B.Cu) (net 5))
 (segment (start 83.225 83.525) (end 81.85 84.9) (width 0.508) (layer B.Cu) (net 5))
 (segment (start 84.35 83.525) (end 83.225 83.525) (width 0.508) (layer B.Cu) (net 5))
 (segment (start 82.6 85.65) (end 81.85 84.9) (width 0.508) (layer B.Cu) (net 5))
 (segment (start 82.6 87.3) (end 82.6 85.65) (width 0.508) (layer B.Cu) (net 5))
 (segment (start 72.79 91.71) (end 72.1 92.4) (width 0.508) (layer B.Cu) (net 14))
 (segment (start 74.65 91.71) (end 72.79 91.71) (width 0.508) (layer B.Cu) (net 14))
 (segment (start 72.25 94.55) (end 72.1 94.4) (width 0.508) (layer B.Cu) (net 14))
 (segment (start 72.25 96.9) (end 72.25 94.55) (width 0.508) (layer B.Cu) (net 14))
 (segment (start 72.1 92.4) (end 72.1 94.4) (width 0.508) (layer B.Cu) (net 14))
 (segment (start 80.39 95.07) (end 79.72 94.4) (width 0.508) (layer B.Cu) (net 19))
 (segment (start 80.39 99.15) (end 80.39 95.07) (width 0.508) (layer B.Cu) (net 19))
 (segment (start 77.6 99.4) (end 77.85 99.15) (width 0.508) (layer B.Cu) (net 17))
 (segment (start 75.45 99.4) (end 77.6 99.4) (width 0.508) (layer B.Cu) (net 17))
 (segment (start 75.56 79.4) (end 75.81 79.15) (width 0.508) (layer B.Cu) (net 18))
 (segment (start 72.6 79.4) (end 75.56 79.4) (width 0.508) (layer B.Cu) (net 18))
 (segment (start 74.89 81.69) (end 72.6 79.4) (width 0.508) (layer B.Cu) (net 18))
 (segment (start 74.89 84.4) (end 74.89 81.69) (width 0.508) (layer B.Cu) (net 18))
 (segment (start 89.2 93.83) (end 91.705 91.325) (width 0.508) (layer B.Cu) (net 16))
 (segment (start 89.2 94.65) (end 89.2 93.83) (width 0.508) (layer B.Cu) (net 16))
 (segment (start 79.6 89.17) (end 81.08 89.17) (width 0.508) (layer B.Cu) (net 4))
 (segment (start 81.08 89.17) (end 81.35 88.9) (width 0.508) (layer B.Cu) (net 4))
 (segment (start 81.35 88.9) (end 83.85 88.9) (width 0.508) (layer B.Cu) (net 4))
 (segment (start 85.1 87.65) (end 85.1 87.3) (width 0.508) (layer B.Cu) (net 4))
 (segment (start 83.85 88.9) (end 85.1 87.65) (width 0.508) (layer B.Cu) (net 4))
 (segment (start 87.6 90.075) (end 87.6 87.9) (width 0.508) (layer B.Cu) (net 4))
 (segment (start 87 87.3) (end 85.1 87.3) (width 0.508) (layer B.Cu) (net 4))
 (segment (start 87.6 87.9) (end 87 87.3) (width 0.508) (layer B.Cu) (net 4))
 (segment (start 85.1 87.3) (end 85.1 87.15) (width 0.508) (layer B.Cu) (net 4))
 (segment (start 86.85 85.4) (end 86.85 83.45) (width 0.508) (layer B.Cu) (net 4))
 (segment (start 85.1 87.15) (end 86.85 85.4) (width 0.508) (layer B.Cu) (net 4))
 (segment (start 87.6 91.345) (end 86.405 91.345) (width 0.508) (layer B.Cu) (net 15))
 (segment (start 86.405 91.345) (end 85.6 92.15) (width 0.508) (layer B.Cu) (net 15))
 (segment (start 85.6 94.15) (end 86.1 94.65) (width 0.508) (layer B.Cu) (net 15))
 (segment (start 85.6 92.15) (end 85.6 94.15) (width 0.508) (layer B.Cu) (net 15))
 (segment (start 74.65 90.44) (end 75.89 90.44) (width 0.508) (layer B.Cu) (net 13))
 (segment (start 75.89 90.44) (end 76.85 91.4) (width 0.508) (layer B.Cu) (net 13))
 (segment (start 76.85 95.4) (end 75.35 96.9) (width 0.508) (layer B.Cu) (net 13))
 (segment (start 76.85 91.4) (end 76.85 95.4) (width 0.508) (layer B.Cu) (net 13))
 (segment (start 75.45 101.65) (end 74.85 101.65) (width 0.508) (layer B.Cu) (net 13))
 (segment (start 74.85 101.65) (end 73.85 100.65) (width 0.508) (layer B.Cu) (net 13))
 (segment (start 73.85 100.65) (end 73.85 97.65) (width 0.508) (layer B.Cu) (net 13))
 (segment (start 74.6 96.9) (end 75.35 96.9) (width 0.508) (layer B.Cu) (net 13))
 (segment (start 73.85 97.65) (end 74.6 96.9) (width 0.508) (layer B.Cu) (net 13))
 (segment (start 94.45 72.95) (end 95.15 72.25) (width 0.508) (layer B.Cu) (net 11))
 (segment (start 94.45 76.55) (end 94.45 72.95) (width 0.508) (layer B.Cu) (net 11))
 (segment (start 93.45 72.25) (end 93.35 72.15) (width 0.508) (layer B.Cu) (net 11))
 (segment (start 95.15 72.25) (end 93.45 72.25) (width 0.508) (layer B.Cu) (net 11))
 (segment (start 82.6 91.6) (end 82.3 91.6) (width 0.508) (layer B.Cu) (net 1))
 (segment (start 81.14 90.44) (end 79.6 90.44) (width 0.508) (layer B.Cu) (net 1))
 (segment (start 82.3 91.6) (end 81.14 90.44) (width 0.508) (layer B.Cu) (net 1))
 (segment (start 82.6 91.6) (end 82.6 90.4) (width 0.508) (layer B.Cu) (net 1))
 (segment (start 85.1 90.4) (end 82.6 90.4) (width 0.508) (layer B.Cu) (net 1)))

